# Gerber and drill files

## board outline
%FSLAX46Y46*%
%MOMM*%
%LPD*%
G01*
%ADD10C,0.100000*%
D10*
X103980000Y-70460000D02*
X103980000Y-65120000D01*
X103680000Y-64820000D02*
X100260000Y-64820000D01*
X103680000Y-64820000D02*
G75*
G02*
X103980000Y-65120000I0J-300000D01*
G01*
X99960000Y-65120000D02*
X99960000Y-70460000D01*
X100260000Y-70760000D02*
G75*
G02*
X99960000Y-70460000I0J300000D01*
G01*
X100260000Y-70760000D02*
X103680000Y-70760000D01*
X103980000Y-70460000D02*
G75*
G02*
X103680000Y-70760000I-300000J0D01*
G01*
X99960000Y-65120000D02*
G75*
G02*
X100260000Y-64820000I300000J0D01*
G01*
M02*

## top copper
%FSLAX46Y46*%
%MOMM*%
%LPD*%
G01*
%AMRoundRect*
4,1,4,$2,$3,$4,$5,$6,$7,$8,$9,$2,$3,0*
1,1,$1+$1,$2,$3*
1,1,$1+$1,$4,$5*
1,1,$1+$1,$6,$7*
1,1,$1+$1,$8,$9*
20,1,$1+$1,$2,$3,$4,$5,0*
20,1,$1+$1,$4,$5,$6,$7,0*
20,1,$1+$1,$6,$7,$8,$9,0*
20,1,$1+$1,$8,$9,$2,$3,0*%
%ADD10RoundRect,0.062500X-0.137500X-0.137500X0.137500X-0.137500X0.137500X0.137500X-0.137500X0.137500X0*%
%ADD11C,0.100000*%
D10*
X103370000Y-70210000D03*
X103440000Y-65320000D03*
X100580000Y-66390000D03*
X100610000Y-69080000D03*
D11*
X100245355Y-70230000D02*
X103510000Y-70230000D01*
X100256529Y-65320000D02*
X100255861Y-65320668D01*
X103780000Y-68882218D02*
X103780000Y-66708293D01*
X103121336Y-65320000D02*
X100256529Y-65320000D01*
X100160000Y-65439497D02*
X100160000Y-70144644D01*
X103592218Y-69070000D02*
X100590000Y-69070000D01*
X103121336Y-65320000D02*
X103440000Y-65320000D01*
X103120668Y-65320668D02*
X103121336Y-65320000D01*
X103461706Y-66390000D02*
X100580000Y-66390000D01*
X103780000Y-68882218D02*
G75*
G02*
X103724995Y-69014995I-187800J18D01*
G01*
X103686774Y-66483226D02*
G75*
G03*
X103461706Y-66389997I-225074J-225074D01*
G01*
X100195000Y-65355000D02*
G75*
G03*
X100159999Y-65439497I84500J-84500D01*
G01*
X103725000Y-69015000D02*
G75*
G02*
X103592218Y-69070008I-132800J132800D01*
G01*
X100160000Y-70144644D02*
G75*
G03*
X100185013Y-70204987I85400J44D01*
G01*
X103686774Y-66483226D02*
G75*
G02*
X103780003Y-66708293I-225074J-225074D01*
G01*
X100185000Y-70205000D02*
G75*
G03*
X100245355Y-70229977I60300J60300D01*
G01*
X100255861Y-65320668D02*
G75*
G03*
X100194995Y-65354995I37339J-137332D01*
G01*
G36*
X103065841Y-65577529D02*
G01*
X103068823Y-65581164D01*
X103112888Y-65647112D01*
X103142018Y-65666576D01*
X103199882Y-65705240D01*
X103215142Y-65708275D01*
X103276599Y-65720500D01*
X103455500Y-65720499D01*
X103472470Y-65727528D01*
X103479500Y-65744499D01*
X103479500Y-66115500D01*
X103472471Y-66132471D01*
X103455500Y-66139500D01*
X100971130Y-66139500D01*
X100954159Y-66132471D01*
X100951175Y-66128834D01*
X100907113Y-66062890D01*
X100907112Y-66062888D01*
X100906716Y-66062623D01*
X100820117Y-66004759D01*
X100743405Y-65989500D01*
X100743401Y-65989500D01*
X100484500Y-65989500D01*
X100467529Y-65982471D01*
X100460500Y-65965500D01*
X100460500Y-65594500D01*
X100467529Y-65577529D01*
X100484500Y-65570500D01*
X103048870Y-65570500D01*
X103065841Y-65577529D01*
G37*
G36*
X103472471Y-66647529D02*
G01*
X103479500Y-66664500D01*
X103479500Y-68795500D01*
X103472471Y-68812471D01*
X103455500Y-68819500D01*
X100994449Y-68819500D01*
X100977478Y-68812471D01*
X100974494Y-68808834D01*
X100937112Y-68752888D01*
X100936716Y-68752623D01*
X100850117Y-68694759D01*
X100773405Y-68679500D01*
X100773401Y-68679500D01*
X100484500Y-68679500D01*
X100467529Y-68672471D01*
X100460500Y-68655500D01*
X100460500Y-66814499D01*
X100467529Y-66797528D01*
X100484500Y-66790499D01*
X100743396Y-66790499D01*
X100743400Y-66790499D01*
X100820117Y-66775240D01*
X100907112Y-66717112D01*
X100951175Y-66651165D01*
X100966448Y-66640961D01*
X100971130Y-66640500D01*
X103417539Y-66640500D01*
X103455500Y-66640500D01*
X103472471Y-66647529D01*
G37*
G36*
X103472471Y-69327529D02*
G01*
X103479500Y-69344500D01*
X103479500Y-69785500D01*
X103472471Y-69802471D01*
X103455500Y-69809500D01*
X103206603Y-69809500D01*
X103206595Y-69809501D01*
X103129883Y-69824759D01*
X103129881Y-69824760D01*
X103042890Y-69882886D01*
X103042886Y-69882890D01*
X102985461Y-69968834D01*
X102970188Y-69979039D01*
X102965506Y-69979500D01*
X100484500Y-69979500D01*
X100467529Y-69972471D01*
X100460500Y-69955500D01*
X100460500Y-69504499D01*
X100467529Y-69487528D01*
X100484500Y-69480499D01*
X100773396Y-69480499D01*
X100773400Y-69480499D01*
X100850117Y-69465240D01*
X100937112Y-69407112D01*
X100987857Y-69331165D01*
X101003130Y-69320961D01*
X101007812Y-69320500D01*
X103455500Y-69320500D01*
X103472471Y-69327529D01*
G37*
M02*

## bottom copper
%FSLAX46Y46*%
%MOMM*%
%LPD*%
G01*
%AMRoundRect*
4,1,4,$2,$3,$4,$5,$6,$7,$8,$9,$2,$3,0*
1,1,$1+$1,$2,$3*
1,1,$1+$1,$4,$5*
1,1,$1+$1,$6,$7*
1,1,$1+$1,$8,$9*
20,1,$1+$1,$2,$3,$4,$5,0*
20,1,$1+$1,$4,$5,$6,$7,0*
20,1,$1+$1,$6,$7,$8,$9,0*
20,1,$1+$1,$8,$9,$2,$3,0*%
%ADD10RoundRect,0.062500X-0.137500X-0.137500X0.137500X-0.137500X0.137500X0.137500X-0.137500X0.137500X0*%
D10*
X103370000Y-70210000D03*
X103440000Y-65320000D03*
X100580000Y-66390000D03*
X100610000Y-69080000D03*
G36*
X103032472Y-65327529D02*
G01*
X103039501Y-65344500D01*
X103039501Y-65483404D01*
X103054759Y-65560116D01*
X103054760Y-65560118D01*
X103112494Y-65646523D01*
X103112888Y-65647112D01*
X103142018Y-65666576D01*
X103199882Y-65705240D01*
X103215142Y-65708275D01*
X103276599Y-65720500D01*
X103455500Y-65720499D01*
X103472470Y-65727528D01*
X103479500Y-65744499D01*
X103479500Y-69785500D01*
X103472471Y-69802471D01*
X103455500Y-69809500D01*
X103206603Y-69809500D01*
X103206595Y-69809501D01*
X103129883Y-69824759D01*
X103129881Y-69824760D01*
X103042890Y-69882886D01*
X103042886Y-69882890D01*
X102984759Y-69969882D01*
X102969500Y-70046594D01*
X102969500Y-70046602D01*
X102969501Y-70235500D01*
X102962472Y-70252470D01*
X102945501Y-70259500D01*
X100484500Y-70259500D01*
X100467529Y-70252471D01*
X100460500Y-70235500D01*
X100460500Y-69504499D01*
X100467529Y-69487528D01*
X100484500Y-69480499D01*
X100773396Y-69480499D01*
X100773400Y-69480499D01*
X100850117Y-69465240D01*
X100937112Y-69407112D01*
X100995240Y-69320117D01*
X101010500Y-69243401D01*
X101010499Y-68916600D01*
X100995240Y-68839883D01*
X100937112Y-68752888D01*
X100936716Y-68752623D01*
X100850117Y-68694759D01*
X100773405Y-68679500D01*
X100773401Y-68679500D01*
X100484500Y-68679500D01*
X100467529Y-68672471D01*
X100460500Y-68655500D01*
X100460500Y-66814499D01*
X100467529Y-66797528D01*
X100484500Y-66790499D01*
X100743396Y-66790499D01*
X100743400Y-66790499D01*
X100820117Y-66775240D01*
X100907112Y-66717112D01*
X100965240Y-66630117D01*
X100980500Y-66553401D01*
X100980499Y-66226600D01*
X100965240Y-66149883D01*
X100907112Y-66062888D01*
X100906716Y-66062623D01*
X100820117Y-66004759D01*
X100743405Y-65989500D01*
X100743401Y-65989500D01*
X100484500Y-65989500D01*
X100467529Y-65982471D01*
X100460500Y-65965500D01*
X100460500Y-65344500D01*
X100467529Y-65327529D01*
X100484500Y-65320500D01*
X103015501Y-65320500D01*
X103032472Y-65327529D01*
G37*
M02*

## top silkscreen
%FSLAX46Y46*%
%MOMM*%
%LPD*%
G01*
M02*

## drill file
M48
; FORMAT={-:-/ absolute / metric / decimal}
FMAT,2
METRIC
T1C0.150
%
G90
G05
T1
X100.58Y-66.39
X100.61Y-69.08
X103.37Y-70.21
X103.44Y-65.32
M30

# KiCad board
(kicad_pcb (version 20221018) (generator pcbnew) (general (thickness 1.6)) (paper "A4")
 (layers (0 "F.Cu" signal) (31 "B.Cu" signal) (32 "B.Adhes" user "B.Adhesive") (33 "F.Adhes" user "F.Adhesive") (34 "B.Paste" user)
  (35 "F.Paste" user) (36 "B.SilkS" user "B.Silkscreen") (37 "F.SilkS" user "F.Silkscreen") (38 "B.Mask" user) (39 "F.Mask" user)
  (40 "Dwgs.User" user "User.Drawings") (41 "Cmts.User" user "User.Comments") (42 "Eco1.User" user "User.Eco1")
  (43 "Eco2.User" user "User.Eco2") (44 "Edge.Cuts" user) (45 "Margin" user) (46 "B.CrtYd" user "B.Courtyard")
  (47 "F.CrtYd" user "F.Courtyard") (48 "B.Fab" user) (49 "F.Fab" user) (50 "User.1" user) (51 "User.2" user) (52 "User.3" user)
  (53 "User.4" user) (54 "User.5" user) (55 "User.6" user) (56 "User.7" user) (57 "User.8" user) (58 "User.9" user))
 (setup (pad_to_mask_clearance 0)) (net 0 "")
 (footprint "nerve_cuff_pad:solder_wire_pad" (layer "F.Cu") (at 103.37 70.21)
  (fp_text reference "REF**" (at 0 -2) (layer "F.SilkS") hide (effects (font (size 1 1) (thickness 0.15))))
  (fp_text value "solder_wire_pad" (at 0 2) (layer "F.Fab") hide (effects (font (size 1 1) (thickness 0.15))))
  (pad "1" thru_hole roundrect (at 0 0) (size 0.4 0.4) (drill 0.15) (layers "*.Cu" "*.Mask") (roundrect_rratio 0.15625)))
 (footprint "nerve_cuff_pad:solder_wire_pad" (layer "F.Cu") (at 103.44 65.32)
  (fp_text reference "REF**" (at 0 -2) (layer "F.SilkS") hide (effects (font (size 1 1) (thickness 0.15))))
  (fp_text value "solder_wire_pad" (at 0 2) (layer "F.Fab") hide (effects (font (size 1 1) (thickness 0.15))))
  (pad "1" thru_hole roundrect (at 0 0) (size 0.4 0.4) (drill 0.15) (layers "*.Cu" "*.Mask") (roundrect_rratio 0.15625)))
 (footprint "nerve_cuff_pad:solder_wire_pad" (layer "F.Cu") (at 100.58 66.39)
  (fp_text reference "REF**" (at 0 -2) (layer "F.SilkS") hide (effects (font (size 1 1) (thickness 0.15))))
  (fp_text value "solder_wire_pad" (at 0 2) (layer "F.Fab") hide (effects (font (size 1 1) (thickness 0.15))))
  (pad "1" thru_hole roundrect (at 0 0) (size 0.4 0.4) (drill 0.15) (layers "*.Cu" "*.Mask") (roundrect_rratio 0.15625)))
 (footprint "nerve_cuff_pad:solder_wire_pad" (layer "F.Cu") (at 100.61 69.08)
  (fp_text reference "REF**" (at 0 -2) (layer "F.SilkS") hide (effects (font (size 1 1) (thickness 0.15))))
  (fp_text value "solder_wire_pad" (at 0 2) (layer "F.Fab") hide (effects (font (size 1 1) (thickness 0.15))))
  (pad "1" thru_hole roundrect (at 0 0) (size 0.4 0.4) (drill 0.15) (layers "*.Cu" "*.Mask") (roundrect_rratio 0.15625)))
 (gr_line (start 103.98 70.46) (end 103.98 65.12) (stroke (width 0.1) (type default)) (layer "Edge.Cuts"))
 (gr_line (start 103.68 64.82) (end 100.26 64.82) (stroke (width 0.1) (type default)) (layer "Edge.Cuts"))
 (gr_arc (start 103.68 64.82) (mid 103.892132 64.907868) (end 103.98 65.12) (stroke (width 0.1) (type default)) (layer "Edge.Cuts"))
 (gr_line (start 99.96 65.12) (end 99.96 70.46) (stroke (width 0.1) (type default)) (layer "Edge.Cuts"))
 (gr_arc (start 100.26 70.76) (mid 100.047868 70.672132) (end 99.96 70.46) (stroke (width 0.1) (type default)) (layer "Edge.Cuts"))
 (gr_line (start 100.26 70.76) (end 103.68 70.76) (stroke (width 0.1) (type default)) (layer "Edge.Cuts"))
 (gr_arc (start 103.98 70.46) (mid 103.892132 70.672132) (end 103.68 70.76) (stroke (width 0.1) (type default)) (layer "Edge.Cuts"))
 (gr_arc (start 99.96 65.12) (mid 100.047868 64.907868) (end 100.26 64.82) (stroke (width 0.1) (type default)) (layer "Edge.Cuts"))
 (segment (start 100.245355 70.23) (end 103.51 70.23) (width 0.1) (layer "F.Cu") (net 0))
 (segment (start 100.256529 65.32) (end 100.255861 65.320668) (width 0.1) (layer "F.Cu") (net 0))
 (segment (start 103.78 68.882218) (end 103.78 66.708293) (width 0.1) (layer "F.Cu") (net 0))
 (segment (start 103.121336 65.32) (end 100.256529 65.32) (width 0.1) (layer "F.Cu") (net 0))
 (segment (start 100.16 65.439497) (end 100.16 70.144644) (width 0.1) (layer "F.Cu") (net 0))
 (segment (start 103.592218 69.07) (end 100.59 69.07) (width 0.1) (layer "F.Cu") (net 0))
 (segment (start 103.121336 65.32) (end 103.44 65.32) (width 0.1) (layer "F.Cu") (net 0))
 (segment (start 103.120668 65.320668) (end 103.121336 65.32) (width 0.1) (layer "F.Cu") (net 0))
 (segment (start 103.461706 66.39) (end 100.58 66.39) (width 0.1) (layer "F.Cu") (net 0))
 (arc (start 103.78 68.882218) (mid 103.765705 68.954079) (end 103.725 69.015) (width 0.1) (layer "F.Cu") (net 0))
 (arc (start 103.686774 66.483226) (mid 103.583512 66.414228) (end 103.461706 66.39) (width 0.1) (layer "F.Cu") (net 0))
 (arc (start 100.195 65.355) (mid 100.169096 65.393767) (end 100.16 65.439497) (width 0.1) (layer "F.Cu") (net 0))
 (arc (start 103.725 69.015) (mid 103.664079 69.055705) (end 103.592218 69.07) (width 0.1) (layer "F.Cu") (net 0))
 (arc (start 100.16 70.144644) (mid 100.166497 70.177308) (end 100.185 70.205) (width 0.1) (layer "F.Cu") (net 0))
 (arc (start 103.686774 66.483226) (mid 103.755771 66.586487) (end 103.78 66.708293) (width 0.1) (layer "F.Cu") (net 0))
 (arc (start 100.185 70.205) (mid 100.212691 70.223508) (end 100.245355 70.23) (width 0.1) (layer "F.Cu") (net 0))
 (arc (start 100.255861 65.320668) (mid 100.223167 65.33411) (end 100.195 65.355) (width 0.1) (layer "F.Cu") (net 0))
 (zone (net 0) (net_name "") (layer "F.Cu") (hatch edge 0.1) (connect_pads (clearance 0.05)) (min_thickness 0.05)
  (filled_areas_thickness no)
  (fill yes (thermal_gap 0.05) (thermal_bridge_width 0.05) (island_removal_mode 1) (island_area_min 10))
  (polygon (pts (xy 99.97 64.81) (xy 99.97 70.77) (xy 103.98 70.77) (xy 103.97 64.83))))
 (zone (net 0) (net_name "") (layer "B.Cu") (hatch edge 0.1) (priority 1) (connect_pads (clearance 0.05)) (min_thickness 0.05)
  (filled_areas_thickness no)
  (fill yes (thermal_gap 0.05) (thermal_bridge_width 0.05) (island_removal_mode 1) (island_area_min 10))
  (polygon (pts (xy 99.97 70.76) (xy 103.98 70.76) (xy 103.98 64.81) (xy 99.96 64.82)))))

